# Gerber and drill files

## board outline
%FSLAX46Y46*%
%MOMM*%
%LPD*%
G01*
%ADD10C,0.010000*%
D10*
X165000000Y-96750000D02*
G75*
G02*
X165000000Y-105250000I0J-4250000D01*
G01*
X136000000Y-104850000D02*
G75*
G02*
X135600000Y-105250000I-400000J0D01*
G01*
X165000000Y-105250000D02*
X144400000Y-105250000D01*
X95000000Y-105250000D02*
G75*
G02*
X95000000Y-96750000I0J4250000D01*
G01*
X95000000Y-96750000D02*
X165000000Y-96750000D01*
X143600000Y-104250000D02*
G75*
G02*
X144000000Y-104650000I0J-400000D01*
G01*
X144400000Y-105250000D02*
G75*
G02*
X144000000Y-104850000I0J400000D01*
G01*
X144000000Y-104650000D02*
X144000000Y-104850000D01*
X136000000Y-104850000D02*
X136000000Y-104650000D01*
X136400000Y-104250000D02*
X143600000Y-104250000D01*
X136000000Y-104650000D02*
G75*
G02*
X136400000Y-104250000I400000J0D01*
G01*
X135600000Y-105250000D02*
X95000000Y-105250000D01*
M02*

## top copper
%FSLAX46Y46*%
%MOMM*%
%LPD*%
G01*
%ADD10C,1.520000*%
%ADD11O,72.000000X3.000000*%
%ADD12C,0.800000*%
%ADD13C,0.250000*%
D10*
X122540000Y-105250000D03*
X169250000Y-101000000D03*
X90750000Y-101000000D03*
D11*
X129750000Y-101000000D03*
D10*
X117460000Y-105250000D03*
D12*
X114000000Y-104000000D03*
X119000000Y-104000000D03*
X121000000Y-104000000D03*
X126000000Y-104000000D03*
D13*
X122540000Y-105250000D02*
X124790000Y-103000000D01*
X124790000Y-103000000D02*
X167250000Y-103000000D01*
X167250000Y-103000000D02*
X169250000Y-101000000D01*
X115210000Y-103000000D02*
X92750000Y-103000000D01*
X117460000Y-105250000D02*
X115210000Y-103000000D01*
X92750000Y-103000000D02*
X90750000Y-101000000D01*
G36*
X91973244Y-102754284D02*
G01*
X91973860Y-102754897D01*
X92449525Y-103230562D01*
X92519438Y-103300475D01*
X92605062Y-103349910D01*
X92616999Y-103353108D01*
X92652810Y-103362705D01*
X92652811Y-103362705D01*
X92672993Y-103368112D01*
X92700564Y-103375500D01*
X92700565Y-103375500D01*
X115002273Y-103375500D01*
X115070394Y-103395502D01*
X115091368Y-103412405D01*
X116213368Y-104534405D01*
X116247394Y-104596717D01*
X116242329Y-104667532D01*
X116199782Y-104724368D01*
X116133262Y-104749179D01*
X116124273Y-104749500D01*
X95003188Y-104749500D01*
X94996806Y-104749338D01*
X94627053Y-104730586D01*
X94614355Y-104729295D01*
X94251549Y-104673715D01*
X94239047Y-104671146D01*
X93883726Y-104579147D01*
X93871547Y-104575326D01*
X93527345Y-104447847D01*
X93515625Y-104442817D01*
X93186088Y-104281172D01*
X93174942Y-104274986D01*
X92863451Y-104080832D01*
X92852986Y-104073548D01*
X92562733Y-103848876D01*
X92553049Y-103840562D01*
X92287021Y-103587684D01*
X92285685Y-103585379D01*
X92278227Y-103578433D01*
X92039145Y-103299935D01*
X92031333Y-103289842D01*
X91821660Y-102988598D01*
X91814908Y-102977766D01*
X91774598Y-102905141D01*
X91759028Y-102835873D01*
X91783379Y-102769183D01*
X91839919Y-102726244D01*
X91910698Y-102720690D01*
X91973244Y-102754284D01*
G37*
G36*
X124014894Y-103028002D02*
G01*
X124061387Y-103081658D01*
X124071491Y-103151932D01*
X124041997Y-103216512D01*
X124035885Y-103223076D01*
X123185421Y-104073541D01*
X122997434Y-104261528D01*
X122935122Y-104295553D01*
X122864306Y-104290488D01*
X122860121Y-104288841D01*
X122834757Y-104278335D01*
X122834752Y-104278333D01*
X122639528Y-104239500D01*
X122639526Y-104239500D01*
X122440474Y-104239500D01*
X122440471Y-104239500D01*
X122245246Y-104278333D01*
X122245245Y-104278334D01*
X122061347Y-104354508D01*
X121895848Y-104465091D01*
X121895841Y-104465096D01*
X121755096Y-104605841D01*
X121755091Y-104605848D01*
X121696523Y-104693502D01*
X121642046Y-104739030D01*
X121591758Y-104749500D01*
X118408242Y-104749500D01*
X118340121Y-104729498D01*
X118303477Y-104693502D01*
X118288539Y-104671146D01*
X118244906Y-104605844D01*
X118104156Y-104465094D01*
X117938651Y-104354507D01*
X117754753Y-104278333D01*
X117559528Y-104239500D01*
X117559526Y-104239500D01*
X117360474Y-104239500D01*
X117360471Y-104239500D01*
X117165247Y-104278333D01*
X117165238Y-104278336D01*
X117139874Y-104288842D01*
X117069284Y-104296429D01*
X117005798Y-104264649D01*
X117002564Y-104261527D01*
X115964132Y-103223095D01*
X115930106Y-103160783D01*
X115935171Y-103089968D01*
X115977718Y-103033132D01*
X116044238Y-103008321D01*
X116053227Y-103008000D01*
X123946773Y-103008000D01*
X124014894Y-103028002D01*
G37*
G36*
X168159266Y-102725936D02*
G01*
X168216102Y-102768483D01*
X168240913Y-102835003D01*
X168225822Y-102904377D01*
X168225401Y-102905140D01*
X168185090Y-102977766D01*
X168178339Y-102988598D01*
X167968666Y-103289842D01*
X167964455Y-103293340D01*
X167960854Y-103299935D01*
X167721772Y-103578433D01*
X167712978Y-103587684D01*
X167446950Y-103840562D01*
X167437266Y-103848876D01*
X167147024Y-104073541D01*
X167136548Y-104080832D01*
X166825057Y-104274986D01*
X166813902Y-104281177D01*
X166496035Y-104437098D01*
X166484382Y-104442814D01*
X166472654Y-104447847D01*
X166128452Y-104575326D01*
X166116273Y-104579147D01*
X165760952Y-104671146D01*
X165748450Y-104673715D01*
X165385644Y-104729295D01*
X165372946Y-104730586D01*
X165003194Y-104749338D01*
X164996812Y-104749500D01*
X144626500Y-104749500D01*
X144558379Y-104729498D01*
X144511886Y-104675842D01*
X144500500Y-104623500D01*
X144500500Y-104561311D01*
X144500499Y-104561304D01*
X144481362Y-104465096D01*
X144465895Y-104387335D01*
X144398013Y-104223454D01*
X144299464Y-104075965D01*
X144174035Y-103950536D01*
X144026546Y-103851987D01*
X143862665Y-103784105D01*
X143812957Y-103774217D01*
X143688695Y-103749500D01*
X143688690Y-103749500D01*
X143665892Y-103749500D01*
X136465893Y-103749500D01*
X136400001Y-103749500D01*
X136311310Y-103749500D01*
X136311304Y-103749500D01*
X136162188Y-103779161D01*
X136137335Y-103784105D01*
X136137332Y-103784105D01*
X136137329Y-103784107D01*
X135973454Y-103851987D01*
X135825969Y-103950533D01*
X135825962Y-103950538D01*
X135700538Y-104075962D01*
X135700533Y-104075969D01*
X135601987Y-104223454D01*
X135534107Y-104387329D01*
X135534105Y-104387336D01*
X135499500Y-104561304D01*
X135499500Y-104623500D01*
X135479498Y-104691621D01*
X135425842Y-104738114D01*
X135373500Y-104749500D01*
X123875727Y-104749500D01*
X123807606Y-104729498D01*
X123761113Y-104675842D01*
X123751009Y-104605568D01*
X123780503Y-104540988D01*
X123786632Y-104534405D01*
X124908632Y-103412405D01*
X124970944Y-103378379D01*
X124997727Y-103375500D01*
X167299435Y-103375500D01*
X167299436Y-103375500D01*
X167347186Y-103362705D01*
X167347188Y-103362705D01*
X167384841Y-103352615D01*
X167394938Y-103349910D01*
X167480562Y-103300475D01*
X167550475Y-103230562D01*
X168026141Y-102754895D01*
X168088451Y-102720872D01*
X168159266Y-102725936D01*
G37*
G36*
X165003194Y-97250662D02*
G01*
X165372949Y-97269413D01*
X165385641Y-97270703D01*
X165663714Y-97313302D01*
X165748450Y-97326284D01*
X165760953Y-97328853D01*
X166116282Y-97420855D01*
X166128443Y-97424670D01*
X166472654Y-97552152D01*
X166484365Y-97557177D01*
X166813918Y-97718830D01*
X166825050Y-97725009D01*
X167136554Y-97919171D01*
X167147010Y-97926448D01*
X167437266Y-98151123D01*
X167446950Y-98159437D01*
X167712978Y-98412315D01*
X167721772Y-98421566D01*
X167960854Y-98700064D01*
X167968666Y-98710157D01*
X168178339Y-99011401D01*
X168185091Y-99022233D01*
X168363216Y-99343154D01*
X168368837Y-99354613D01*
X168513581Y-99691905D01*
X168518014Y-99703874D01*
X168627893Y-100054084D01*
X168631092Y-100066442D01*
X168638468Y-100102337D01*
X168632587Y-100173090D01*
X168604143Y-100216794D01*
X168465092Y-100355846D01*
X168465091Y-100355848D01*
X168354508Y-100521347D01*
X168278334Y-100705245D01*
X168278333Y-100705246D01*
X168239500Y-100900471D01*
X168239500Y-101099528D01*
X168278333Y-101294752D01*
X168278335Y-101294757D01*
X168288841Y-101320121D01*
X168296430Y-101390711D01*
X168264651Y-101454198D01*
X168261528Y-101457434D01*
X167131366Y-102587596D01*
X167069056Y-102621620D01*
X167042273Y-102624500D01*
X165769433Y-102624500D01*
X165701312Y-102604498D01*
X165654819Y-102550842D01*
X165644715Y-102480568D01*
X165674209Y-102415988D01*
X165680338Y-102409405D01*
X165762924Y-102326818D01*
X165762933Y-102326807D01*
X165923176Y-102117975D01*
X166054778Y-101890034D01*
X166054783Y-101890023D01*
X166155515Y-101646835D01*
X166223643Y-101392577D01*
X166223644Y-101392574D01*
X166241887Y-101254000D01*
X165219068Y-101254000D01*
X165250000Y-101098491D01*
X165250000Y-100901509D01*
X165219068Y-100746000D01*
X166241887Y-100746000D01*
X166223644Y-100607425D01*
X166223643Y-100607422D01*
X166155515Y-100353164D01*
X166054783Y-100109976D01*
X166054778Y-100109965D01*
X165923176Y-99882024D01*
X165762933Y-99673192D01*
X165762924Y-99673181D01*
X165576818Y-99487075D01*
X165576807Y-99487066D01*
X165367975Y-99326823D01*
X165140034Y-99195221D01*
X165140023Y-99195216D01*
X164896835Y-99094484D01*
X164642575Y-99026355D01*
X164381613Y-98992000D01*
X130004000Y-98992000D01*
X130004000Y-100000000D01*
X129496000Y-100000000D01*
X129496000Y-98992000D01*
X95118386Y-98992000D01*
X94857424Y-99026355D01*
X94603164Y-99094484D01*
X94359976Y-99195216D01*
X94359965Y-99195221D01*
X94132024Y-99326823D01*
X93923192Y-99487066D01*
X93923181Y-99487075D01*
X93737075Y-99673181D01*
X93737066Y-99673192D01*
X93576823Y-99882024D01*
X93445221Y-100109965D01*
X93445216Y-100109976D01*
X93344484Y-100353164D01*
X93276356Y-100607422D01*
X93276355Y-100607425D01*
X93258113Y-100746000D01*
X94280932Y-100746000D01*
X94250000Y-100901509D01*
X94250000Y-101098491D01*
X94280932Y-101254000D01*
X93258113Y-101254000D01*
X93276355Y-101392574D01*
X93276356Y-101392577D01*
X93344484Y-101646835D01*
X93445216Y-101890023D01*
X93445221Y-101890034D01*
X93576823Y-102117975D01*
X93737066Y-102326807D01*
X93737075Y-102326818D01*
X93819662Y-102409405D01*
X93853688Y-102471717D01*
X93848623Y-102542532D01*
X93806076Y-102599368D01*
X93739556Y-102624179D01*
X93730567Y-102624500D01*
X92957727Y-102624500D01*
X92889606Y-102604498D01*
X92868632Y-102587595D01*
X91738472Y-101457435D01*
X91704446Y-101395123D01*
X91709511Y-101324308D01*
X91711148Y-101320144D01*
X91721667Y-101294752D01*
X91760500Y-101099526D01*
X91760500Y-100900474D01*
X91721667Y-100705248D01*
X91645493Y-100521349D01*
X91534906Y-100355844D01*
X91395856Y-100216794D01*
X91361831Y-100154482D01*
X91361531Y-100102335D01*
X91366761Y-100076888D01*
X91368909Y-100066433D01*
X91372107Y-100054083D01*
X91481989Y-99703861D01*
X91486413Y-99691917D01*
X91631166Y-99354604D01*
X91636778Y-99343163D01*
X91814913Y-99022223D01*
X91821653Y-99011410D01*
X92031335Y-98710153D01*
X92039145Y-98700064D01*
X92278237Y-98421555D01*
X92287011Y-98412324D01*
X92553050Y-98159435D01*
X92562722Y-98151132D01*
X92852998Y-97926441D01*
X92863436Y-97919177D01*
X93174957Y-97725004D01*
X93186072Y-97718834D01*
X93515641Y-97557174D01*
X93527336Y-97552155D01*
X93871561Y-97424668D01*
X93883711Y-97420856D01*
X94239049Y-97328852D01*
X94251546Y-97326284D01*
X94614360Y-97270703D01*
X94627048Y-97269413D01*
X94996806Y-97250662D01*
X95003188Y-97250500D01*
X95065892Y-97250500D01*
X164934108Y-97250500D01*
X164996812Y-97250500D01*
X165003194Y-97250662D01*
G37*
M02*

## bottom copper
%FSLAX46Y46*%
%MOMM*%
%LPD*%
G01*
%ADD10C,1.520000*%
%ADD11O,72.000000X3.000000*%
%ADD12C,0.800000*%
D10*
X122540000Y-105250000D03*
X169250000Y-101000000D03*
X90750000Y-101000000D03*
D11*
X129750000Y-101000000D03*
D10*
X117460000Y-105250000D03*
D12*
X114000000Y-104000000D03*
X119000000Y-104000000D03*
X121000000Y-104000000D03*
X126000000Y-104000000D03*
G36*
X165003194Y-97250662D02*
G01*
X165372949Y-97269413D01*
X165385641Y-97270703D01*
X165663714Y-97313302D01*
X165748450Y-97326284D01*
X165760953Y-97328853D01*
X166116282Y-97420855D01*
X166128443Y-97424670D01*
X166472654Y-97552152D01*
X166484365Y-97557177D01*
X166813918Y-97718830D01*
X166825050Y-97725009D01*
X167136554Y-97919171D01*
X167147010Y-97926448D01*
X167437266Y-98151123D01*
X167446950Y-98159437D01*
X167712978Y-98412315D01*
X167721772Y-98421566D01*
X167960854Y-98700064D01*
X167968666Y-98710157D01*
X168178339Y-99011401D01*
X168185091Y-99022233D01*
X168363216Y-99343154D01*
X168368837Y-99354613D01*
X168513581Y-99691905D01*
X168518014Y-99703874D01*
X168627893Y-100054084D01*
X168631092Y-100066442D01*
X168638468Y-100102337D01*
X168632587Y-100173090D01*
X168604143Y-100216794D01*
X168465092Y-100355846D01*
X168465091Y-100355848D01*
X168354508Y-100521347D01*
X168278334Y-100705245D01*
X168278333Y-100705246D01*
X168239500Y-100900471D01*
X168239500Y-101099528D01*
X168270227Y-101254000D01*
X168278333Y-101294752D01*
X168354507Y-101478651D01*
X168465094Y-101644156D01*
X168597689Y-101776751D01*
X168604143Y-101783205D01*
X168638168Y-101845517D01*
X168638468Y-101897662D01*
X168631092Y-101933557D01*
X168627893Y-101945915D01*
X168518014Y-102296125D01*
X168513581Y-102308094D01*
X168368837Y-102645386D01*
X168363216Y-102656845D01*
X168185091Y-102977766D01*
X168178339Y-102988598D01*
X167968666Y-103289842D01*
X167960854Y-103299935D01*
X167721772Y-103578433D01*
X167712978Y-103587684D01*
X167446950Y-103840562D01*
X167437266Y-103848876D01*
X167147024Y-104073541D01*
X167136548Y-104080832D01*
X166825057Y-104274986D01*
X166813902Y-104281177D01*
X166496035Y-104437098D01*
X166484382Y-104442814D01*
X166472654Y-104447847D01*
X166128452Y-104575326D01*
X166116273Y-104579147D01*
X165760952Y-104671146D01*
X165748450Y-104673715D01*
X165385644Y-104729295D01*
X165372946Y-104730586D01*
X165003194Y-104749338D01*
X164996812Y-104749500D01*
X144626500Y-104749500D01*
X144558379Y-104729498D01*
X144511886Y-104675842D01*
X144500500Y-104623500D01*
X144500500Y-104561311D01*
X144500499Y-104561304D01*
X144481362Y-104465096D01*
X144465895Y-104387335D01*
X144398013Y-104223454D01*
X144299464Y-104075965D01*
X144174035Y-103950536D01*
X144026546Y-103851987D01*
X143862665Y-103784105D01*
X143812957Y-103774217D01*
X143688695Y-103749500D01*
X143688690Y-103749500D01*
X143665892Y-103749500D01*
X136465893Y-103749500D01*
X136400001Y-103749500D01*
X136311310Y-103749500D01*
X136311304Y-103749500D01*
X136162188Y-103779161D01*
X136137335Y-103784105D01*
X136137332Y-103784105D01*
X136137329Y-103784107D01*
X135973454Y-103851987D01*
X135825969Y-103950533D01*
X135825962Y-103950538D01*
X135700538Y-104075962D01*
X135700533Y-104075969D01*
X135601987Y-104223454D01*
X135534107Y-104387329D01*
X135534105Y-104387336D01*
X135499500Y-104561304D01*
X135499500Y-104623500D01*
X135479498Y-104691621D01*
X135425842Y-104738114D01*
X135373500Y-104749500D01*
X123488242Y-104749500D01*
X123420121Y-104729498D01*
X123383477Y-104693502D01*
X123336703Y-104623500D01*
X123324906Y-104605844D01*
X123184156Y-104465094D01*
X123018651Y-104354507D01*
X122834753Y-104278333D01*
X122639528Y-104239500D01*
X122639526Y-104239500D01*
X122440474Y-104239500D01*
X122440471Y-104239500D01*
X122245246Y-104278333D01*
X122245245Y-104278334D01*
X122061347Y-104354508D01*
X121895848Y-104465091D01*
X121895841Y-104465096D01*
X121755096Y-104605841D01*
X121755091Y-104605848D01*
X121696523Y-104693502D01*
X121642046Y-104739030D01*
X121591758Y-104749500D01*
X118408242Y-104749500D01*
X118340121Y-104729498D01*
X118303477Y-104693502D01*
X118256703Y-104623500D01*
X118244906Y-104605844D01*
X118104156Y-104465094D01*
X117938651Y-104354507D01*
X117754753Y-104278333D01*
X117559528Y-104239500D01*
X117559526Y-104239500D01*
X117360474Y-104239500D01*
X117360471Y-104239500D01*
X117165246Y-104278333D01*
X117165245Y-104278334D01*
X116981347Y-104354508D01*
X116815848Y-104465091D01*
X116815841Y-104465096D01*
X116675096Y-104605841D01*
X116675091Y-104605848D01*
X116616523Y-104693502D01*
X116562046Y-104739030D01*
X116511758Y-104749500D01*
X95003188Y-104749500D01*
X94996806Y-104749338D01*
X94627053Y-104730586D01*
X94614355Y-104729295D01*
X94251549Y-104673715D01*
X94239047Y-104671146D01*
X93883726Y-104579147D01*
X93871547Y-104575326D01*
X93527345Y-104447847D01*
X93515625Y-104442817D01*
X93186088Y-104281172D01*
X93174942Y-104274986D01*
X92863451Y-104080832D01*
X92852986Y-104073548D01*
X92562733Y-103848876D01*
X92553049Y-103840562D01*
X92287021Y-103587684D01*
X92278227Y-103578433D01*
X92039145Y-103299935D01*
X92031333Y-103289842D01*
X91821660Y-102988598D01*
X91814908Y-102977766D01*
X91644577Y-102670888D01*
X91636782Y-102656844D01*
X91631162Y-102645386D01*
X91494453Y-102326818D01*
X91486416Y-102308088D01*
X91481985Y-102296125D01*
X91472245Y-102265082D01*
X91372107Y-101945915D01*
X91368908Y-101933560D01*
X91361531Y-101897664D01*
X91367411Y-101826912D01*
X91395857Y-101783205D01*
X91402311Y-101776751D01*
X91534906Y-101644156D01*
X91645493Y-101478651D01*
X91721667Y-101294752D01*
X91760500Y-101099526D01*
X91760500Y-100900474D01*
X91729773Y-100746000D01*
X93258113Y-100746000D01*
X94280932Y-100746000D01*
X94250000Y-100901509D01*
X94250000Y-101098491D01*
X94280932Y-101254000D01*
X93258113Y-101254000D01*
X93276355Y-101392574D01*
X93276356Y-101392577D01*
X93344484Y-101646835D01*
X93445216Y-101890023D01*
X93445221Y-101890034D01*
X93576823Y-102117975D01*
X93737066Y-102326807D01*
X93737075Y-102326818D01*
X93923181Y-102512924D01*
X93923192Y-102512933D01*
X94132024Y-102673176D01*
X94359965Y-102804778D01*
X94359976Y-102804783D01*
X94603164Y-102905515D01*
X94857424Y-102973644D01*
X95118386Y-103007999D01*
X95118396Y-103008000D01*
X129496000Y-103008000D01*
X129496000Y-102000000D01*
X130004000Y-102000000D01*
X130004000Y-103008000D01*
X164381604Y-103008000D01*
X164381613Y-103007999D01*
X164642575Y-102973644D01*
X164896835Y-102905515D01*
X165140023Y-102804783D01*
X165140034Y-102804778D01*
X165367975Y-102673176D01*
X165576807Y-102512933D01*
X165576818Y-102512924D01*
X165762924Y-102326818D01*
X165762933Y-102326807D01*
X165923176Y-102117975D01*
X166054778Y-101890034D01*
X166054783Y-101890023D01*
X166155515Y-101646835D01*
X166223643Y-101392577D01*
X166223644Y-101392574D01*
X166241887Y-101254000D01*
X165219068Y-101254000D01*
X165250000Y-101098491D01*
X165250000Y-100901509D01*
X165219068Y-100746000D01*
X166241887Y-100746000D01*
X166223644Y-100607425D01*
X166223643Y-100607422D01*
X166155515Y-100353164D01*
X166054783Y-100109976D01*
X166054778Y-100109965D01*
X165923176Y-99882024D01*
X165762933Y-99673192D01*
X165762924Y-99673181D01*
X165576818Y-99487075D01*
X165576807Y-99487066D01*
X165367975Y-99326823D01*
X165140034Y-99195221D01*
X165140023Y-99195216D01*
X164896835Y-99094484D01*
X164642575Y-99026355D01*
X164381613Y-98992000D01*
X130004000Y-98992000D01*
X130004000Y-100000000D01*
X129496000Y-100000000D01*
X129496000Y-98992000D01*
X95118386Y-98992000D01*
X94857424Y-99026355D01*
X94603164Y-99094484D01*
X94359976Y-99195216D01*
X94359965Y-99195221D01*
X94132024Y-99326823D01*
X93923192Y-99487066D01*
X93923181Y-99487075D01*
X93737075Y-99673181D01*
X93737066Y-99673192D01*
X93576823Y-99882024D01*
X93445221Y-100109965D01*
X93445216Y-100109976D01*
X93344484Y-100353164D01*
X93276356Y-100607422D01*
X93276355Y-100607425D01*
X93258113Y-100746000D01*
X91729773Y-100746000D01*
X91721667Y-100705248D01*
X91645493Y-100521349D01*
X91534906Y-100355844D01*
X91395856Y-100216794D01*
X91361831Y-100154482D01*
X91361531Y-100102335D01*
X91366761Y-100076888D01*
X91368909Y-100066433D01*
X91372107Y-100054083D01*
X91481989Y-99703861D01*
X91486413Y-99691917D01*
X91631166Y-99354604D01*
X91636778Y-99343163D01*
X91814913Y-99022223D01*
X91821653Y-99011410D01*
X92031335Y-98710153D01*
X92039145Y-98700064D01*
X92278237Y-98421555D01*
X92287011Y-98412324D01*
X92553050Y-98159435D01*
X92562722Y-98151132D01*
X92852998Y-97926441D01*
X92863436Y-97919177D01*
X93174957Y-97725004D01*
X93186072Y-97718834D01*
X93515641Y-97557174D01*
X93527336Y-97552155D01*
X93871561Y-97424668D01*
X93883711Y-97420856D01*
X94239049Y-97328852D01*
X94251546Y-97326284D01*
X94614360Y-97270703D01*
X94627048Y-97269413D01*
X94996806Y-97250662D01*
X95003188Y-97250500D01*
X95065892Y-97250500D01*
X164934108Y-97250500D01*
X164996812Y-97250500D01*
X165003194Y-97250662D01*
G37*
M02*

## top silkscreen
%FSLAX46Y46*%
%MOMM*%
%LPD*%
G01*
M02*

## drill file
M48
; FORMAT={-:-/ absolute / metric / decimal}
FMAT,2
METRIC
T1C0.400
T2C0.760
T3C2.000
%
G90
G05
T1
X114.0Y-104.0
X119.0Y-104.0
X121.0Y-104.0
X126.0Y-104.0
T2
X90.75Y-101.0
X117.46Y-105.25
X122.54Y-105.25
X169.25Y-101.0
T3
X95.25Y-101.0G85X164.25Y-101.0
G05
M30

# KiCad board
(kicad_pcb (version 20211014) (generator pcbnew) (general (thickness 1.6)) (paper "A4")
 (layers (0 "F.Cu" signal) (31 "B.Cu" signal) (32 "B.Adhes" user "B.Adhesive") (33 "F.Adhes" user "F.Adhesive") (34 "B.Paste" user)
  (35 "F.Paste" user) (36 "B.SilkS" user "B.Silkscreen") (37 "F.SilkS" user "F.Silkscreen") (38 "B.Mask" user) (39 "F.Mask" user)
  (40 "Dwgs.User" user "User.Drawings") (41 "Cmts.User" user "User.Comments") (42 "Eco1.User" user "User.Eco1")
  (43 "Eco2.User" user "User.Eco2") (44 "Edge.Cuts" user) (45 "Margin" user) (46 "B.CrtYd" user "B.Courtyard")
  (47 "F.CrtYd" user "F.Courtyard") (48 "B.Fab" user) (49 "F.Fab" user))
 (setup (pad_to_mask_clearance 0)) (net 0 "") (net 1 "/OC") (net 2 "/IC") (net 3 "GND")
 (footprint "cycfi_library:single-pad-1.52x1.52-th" (layer "F.Cu") (at 122.54 105.25 180)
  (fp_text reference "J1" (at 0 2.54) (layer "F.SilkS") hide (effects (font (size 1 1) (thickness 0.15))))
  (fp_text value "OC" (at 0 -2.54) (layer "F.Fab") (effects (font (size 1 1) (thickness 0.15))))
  (pad "1" thru_hole circle (at 0 0 180) (size 1.52 1.52) (drill 0.76) (layers *.Cu *.Mask) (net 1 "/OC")))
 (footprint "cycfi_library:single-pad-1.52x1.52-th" (layer "F.Cu") (at 169.25 101 180)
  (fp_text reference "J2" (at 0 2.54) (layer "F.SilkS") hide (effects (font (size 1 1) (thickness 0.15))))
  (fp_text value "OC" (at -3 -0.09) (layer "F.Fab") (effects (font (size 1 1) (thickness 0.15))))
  (pad "1" thru_hole circle (at 0 0 180) (size 1.52 1.52) (drill 0.76) (layers *.Cu *.Mask) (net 1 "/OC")))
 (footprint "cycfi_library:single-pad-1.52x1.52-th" (layer "F.Cu") (at 90.75 101)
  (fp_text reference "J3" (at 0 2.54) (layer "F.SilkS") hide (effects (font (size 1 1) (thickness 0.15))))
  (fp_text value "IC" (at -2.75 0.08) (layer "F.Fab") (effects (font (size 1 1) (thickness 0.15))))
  (pad "1" thru_hole circle (at 0 0) (size 1.52 1.52) (drill 0.76) (layers *.Cu *.Mask) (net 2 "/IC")))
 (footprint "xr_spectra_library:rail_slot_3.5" (layer "F.Cu") (at 129.75 101)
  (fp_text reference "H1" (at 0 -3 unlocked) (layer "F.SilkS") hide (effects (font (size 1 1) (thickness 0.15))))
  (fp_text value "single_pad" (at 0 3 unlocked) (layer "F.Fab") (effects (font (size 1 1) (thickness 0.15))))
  (pad "1" thru_hole oval (at 0 0) (size 72 3) (drill oval 71 2) (layers *.Cu "B.Mask") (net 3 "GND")))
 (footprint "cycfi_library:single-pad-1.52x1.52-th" (layer "F.Cu") (at 117.46 105.25)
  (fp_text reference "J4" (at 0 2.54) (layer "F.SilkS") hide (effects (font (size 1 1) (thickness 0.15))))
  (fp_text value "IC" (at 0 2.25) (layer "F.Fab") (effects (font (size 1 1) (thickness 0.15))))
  (pad "1" thru_hole circle (at 0 0) (size 1.52 1.52) (drill 0.76) (layers *.Cu *.Mask) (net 2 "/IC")))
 (gr_arc (start 165 96.75) (mid 169.25 101) (end 165 105.25) (layer "Edge.Cuts") (width 0.01))
 (gr_arc (start 136 104.85) (mid 135.882843 105.132843) (end 135.6 105.25) (layer "Edge.Cuts") (width 0.01))
 (gr_line (start 165 105.25) (end 144.4 105.25) (layer "Edge.Cuts") (width 0.01))
 (gr_arc (start 95 105.25) (mid 90.75 101) (end 95 96.75) (layer "Edge.Cuts") (width 0.01))
 (gr_line (start 95 96.75) (end 165 96.75) (layer "Edge.Cuts") (width 0.01))
 (gr_arc (start 143.6 104.25) (mid 143.882843 104.367157) (end 144 104.65) (layer "Edge.Cuts") (width 0.01))
 (gr_arc (start 144.4 105.25) (mid 144.117157 105.132843) (end 144 104.85) (layer "Edge.Cuts") (width 0.01))
 (gr_line (start 144 104.65) (end 144 104.85) (layer "Edge.Cuts") (width 0.01))
 (gr_line (start 136 104.85) (end 136 104.65) (layer "Edge.Cuts") (width 0.01))
 (gr_line (start 136.4 104.25) (end 143.6 104.25) (layer "Edge.Cuts") (width 0.01))
 (gr_arc (start 136 104.65) (mid 136.117157 104.367157) (end 136.4 104.25) (layer "Edge.Cuts") (width 0.01))
 (gr_line (start 135.6 105.25) (end 95 105.25) (layer "Edge.Cuts") (width 0.01))
 (via (at 114 104) (size 0.8) (drill 0.4) (layers "F.Cu" "B.Cu") (free) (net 3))
 (via (at 119 104) (size 0.8) (drill 0.4) (layers "F.Cu" "B.Cu") (free) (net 3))
 (via (at 121 104) (size 0.8) (drill 0.4) (layers "F.Cu" "B.Cu") (free) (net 3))
 (via (at 126 104) (size 0.8) (drill 0.4) (layers "F.Cu" "B.Cu") (free) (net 3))
 (segment (start 122.54 105.25) (end 124.79 103) (width 0.25) (layer "F.Cu") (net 1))
 (segment (start 124.79 103) (end 167.25 103) (width 0.25) (layer "F.Cu") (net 1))
 (segment (start 167.25 103) (end 169.25 101) (width 0.25) (layer "F.Cu") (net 1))
 (segment (start 115.21 103) (end 92.75 103) (width 0.25) (layer "F.Cu") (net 2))
 (segment (start 117.46 105.25) (end 115.21 103) (width 0.25) (layer "F.Cu") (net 2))
 (segment (start 92.75 103) (end 90.75 101) (width 0.25) (layer "F.Cu") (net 2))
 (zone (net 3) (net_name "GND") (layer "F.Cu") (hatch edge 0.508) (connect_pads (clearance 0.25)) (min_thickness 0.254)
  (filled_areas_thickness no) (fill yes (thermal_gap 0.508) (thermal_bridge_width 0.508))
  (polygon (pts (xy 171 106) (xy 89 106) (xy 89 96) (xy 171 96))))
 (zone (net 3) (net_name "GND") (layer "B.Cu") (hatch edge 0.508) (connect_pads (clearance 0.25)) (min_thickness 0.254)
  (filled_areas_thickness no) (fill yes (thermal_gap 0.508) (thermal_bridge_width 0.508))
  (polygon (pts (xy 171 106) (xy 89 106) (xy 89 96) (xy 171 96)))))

